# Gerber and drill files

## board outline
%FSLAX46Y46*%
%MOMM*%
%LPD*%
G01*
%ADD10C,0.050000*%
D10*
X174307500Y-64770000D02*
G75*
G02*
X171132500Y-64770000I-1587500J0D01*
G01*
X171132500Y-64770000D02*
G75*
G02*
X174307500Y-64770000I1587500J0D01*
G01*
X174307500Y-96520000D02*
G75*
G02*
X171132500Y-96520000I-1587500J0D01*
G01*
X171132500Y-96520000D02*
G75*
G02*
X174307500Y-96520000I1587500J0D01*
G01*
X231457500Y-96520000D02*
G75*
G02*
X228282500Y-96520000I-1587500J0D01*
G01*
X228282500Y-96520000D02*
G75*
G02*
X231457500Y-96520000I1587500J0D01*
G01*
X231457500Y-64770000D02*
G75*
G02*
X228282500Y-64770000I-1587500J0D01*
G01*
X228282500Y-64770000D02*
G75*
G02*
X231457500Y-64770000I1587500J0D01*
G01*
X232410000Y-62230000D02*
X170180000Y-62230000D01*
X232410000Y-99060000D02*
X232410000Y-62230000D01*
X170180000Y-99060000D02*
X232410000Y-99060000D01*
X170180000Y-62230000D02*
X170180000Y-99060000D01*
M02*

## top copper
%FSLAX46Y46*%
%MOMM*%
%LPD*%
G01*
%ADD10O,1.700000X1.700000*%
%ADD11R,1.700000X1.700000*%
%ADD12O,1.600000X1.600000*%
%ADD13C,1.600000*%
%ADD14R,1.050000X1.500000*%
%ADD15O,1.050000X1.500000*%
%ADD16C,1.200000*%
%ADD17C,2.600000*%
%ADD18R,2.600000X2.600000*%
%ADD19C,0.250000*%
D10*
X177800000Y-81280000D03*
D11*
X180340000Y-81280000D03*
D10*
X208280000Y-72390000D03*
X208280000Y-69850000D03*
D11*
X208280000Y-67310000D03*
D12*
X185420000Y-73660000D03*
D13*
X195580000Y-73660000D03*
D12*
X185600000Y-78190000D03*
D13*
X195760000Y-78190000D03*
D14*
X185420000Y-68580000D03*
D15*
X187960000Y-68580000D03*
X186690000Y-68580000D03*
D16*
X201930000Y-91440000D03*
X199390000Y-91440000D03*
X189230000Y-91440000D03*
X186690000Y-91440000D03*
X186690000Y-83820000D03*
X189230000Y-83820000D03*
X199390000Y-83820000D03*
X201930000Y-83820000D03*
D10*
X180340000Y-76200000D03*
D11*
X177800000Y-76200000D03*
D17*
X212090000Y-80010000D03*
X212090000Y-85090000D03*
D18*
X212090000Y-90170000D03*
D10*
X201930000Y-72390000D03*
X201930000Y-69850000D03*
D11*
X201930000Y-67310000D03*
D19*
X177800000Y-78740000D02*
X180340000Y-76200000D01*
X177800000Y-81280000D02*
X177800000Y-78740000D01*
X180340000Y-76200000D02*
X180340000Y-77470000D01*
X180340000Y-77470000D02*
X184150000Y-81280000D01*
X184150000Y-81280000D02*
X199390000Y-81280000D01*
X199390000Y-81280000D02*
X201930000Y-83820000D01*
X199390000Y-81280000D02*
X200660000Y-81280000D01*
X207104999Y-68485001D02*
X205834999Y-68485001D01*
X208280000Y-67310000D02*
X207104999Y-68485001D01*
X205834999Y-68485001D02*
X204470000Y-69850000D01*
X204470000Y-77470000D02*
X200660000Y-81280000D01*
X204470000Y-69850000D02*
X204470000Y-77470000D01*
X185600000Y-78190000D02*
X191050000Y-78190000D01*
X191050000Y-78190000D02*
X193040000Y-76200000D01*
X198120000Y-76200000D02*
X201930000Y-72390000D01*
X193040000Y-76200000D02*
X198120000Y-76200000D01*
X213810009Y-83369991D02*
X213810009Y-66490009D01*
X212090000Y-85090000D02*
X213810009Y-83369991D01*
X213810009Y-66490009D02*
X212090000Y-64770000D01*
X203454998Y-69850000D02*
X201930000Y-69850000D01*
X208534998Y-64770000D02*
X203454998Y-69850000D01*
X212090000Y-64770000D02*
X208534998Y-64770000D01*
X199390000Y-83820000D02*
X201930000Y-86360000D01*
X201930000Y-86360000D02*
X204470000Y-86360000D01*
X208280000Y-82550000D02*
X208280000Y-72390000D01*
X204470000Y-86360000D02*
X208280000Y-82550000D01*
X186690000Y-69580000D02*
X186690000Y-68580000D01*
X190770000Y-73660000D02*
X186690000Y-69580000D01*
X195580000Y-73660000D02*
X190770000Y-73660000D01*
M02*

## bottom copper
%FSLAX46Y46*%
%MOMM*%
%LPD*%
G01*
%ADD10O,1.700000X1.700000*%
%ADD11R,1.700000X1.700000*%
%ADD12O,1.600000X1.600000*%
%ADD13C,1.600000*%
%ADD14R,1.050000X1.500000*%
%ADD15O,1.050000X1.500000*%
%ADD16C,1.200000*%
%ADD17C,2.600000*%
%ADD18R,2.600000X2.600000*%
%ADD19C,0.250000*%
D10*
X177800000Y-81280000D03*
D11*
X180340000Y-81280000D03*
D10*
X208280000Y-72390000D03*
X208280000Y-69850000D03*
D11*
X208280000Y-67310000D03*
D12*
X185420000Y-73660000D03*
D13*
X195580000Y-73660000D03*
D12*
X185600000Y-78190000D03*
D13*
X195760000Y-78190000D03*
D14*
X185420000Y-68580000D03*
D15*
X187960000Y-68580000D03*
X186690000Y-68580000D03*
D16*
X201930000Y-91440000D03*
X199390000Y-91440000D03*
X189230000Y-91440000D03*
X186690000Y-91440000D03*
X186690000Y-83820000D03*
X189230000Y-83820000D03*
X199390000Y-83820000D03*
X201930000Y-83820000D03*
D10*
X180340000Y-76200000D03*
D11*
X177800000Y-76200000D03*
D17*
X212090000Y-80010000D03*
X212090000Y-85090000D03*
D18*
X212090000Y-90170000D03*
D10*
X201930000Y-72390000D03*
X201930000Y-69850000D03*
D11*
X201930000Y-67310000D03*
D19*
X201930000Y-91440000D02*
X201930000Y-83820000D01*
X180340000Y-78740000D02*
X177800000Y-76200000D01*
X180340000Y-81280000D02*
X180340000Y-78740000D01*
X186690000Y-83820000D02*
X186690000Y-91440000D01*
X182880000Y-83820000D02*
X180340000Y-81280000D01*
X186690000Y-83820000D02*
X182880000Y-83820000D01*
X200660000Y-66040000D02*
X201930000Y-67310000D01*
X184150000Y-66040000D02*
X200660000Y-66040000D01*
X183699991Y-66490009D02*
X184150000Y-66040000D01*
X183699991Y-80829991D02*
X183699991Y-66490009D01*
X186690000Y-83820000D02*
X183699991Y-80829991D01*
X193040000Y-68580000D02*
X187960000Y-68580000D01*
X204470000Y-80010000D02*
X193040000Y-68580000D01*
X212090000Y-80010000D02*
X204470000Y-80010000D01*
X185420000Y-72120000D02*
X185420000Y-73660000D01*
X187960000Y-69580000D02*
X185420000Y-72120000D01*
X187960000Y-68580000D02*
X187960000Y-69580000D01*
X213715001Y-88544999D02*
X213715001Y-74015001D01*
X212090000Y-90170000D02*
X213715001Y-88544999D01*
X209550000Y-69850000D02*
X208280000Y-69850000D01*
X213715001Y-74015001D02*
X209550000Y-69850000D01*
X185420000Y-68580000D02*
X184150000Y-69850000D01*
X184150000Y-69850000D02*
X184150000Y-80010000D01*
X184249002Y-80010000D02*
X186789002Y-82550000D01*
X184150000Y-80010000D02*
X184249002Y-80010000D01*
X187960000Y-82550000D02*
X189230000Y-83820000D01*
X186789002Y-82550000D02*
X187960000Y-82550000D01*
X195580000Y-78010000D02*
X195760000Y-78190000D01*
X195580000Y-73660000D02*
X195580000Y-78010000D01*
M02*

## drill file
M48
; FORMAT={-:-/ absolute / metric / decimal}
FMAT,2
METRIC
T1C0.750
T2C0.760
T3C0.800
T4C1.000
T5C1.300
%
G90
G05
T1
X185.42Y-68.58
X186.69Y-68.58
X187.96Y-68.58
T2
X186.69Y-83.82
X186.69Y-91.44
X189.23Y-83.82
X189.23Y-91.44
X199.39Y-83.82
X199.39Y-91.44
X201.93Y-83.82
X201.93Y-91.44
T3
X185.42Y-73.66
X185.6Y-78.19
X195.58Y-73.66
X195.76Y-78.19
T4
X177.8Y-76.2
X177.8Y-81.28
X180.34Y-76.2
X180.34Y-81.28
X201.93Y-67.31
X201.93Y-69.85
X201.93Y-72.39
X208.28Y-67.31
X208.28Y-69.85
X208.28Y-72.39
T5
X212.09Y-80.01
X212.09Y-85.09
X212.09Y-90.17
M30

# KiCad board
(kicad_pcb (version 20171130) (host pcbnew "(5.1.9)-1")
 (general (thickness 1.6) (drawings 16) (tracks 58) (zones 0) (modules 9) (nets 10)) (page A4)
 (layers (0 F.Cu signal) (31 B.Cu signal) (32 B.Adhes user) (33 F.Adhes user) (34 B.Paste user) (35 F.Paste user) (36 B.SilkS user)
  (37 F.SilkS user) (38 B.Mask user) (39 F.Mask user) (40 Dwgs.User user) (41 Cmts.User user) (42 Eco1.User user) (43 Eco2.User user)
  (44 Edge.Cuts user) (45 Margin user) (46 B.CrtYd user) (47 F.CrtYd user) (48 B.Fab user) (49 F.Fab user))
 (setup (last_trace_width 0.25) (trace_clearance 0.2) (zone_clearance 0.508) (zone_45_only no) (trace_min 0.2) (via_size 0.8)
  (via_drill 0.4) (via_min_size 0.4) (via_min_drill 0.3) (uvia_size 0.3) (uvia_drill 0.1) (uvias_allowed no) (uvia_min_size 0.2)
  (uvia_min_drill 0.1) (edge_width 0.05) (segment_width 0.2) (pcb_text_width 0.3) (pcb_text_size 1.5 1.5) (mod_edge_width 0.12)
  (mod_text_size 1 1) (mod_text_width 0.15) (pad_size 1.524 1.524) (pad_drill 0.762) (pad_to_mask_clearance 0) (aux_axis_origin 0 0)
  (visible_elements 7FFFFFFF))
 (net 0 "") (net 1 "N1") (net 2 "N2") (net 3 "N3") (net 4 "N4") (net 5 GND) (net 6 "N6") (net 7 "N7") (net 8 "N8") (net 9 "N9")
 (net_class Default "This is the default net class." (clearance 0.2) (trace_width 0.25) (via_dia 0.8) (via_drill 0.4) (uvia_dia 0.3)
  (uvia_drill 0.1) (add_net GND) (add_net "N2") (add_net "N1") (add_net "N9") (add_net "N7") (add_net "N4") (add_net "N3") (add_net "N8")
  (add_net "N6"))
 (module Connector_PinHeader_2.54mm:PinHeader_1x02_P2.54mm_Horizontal (layer F.Cu) (at 180.34 81.28 270)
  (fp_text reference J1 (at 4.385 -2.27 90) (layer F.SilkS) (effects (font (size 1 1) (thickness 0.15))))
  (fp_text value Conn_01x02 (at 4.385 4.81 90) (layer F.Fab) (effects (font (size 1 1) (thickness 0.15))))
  (pad 2 thru_hole oval (at 0 2.54 270) (size 1.7 1.7) (drill 1) (layers *.Cu *.Mask) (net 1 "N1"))
  (pad 1 thru_hole rect (at 0 0 270) (size 1.7 1.7) (drill 1) (layers *.Cu *.Mask) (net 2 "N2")))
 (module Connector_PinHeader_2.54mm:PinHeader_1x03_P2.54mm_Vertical (layer F.Cu) (at 208.28 67.31)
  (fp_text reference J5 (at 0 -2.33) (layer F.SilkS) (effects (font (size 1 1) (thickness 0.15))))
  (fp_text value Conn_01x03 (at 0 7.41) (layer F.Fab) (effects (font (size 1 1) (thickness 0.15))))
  (pad 3 thru_hole oval (at 0 5.08) (size 1.7 1.7) (drill 1) (layers *.Cu *.Mask) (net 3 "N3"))
  (pad 2 thru_hole oval (at 0 2.54) (size 1.7 1.7) (drill 1) (layers *.Cu *.Mask) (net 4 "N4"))
  (pad 1 thru_hole rect (at 0 0) (size 1.7 1.7) (drill 1) (layers *.Cu *.Mask) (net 1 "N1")))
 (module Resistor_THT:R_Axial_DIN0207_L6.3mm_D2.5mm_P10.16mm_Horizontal (layer F.Cu) (at 195.58 73.66 180)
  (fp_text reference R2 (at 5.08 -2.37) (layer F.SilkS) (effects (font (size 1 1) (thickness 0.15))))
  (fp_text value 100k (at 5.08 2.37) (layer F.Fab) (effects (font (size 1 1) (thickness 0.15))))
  (pad 2 thru_hole oval (at 10.16 0 180) (size 1.6 1.6) (drill 0.8) (layers *.Cu *.Mask) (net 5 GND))
  (pad 1 thru_hole circle (at 0 0 180) (size 1.6 1.6) (drill 0.8) (layers *.Cu *.Mask) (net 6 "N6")))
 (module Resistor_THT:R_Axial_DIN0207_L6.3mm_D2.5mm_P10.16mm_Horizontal (layer F.Cu) (at 195.76 78.19 180)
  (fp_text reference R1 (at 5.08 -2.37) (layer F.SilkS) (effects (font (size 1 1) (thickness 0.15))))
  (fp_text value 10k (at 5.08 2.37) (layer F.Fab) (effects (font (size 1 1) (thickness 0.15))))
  (pad 2 thru_hole oval (at 10.16 0 180) (size 1.6 1.6) (drill 0.8) (layers *.Cu *.Mask) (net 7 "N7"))
  (pad 1 thru_hole circle (at 0 0 180) (size 1.6 1.6) (drill 0.8) (layers *.Cu *.Mask) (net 6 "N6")))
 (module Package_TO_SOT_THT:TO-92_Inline (layer F.Cu) (at 185.42 68.58)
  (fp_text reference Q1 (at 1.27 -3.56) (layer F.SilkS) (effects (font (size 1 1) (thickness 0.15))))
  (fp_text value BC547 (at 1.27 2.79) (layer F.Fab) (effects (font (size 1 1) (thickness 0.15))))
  (pad 1 thru_hole rect (at 0 0) (size 1.05 1.5) (drill 0.75) (layers *.Cu *.Mask) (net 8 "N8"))
  (pad 3 thru_hole oval (at 2.54 0) (size 1.05 1.5) (drill 0.75) (layers *.Cu *.Mask) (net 5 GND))
  (pad 2 thru_hole oval (at 1.27 0) (size 1.05 1.5) (drill 0.75) (layers *.Cu *.Mask) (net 6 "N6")))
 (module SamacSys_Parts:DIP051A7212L (layer F.Cu) (at 201.93 83.82 180)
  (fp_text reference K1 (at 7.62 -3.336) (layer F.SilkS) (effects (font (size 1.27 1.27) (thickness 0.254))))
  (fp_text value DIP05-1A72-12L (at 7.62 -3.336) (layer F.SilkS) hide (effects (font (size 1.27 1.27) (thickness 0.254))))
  (pad 14 thru_hole circle (at 0 -7.62 180) (size 1.2 1.2) (drill 0.76) (layers *.Cu *.Mask) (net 1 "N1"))
  (pad 13 thru_hole circle (at 2.54 -7.62 180) (size 1.2 1.2) (drill 0.76) (layers *.Cu *.Mask))
  (pad 9 thru_hole circle (at 12.7 -7.62 180) (size 1.2 1.2) (drill 0.76) (layers *.Cu *.Mask))
  (pad 8 thru_hole circle (at 15.24 -7.62 180) (size 1.2 1.2) (drill 0.76) (layers *.Cu *.Mask) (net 2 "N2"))
  (pad 7 thru_hole circle (at 15.24 0 180) (size 1.2 1.2) (drill 0.76) (layers *.Cu *.Mask) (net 2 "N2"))
  (pad 6 thru_hole circle (at 12.7 0 180) (size 1.2 1.2) (drill 0.76) (layers *.Cu *.Mask) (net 8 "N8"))
  (pad 2 thru_hole circle (at 2.54 0 180) (size 1.2 1.2) (drill 0.76) (layers *.Cu *.Mask) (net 3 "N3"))
  (pad 1 thru_hole circle (at 0 0 180) (size 1.2 1.2) (drill 0.76) (layers *.Cu *.Mask) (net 1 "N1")))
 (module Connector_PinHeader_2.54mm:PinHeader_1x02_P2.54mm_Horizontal (layer F.Cu) (at 177.8 76.2 90)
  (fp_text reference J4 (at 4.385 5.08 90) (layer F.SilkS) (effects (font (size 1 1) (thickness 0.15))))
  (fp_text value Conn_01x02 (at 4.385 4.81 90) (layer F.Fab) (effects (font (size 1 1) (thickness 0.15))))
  (pad 2 thru_hole oval (at 0 2.54 90) (size 1.7 1.7) (drill 1) (layers *.Cu *.Mask) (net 1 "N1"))
  (pad 1 thru_hole rect (at 0 0 90) (size 1.7 1.7) (drill 1) (layers *.Cu *.Mask) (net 2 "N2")))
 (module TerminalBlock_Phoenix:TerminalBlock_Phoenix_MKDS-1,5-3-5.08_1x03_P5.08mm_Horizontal (layer F.Cu) (at 212.09 90.17 90)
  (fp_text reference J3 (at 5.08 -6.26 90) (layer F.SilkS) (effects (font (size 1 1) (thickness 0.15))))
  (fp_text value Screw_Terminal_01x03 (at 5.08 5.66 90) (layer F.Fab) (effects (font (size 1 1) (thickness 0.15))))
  (pad 3 thru_hole circle (at 10.16 0 90) (size 2.6 2.6) (drill 1.3) (layers *.Cu *.Mask) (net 5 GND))
  (pad 2 thru_hole circle (at 5.08 0 90) (size 2.6 2.6) (drill 1.3) (layers *.Cu *.Mask) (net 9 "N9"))
  (pad 1 thru_hole rect (at 0 0 90) (size 2.6 2.6) (drill 1.3) (layers *.Cu *.Mask) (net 4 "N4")))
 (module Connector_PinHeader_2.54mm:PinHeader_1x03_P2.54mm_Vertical (layer F.Cu) (at 201.93 67.31)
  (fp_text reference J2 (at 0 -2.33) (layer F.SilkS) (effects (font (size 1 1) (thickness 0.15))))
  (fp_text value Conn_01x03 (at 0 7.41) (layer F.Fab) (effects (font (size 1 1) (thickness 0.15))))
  (pad 3 thru_hole oval (at 0 5.08) (size 1.7 1.7) (drill 1) (layers *.Cu *.Mask) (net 7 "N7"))
  (pad 2 thru_hole oval (at 0 2.54) (size 1.7 1.7) (drill 1) (layers *.Cu *.Mask) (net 9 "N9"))
  (pad 1 thru_hole rect (at 0 0) (size 1.7 1.7) (drill 1) (layers *.Cu *.Mask) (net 2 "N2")))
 (gr_circle (center 172.72 64.77) (end 174.3075 64.77) (layer Edge.Cuts) (width 0.05))
 (gr_circle (center 172.72 96.52) (end 174.3075 96.52) (layer Edge.Cuts) (width 0.05))
 (gr_circle (center 229.87 96.52) (end 231.4575 96.52) (layer Edge.Cuts) (width 0.05))
 (gr_circle (center 229.87 64.77) (end 231.4575 64.77) (layer Edge.Cuts) (width 0.05))
 (gr_line (start 232.41 62.23) (end 170.18 62.23) (layer Edge.Cuts) (width 0.05))
 (gr_line (start 232.41 99.06) (end 232.41 62.23) (layer Edge.Cuts) (width 0.05))
 (gr_line (start 170.18 99.06) (end 232.41 99.06) (layer Edge.Cuts) (width 0.05))
 (gr_line (start 170.18 62.23) (end 170.18 99.06) (layer Edge.Cuts) (width 0.05))
 (segment (start 177.8 78.74) (end 180.34 76.2) (width 0.25) (layer F.Cu) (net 1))
 (segment (start 177.8 81.28) (end 177.8 78.74) (width 0.25) (layer F.Cu) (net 1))
 (segment (start 201.93 91.44) (end 201.93 83.82) (width 0.25) (layer B.Cu) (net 1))
 (segment (start 180.34 76.2) (end 180.34 77.47) (width 0.25) (layer F.Cu) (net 1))
 (segment (start 180.34 77.47) (end 184.15 81.28) (width 0.25) (layer F.Cu) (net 1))
 (segment (start 184.15 81.28) (end 199.39 81.28) (width 0.25) (layer F.Cu) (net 1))
 (segment (start 199.39 81.28) (end 201.93 83.82) (width 0.25) (layer F.Cu) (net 1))
 (segment (start 199.39 81.28) (end 200.66 81.28) (width 0.25) (layer F.Cu) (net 1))
 (segment (start 207.104999 68.485001) (end 205.834999 68.485001) (width 0.25) (layer F.Cu) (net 1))
 (segment (start 208.28 67.31) (end 207.104999 68.485001) (width 0.25) (layer F.Cu) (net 1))
 (segment (start 205.834999 68.485001) (end 204.47 69.85) (width 0.25) (layer F.Cu) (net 1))
 (segment (start 204.47 77.47) (end 200.66 81.28) (width 0.25) (layer F.Cu) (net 1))
 (segment (start 204.47 69.85) (end 204.47 77.47) (width 0.25) (layer F.Cu) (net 1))
 (segment (start 180.34 78.74) (end 177.8 76.2) (width 0.25) (layer B.Cu) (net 2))
 (segment (start 180.34 81.28) (end 180.34 78.74) (width 0.25) (layer B.Cu) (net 2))
 (segment (start 186.69 83.82) (end 186.69 91.44) (width 0.25) (layer B.Cu) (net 2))
 (segment (start 182.88 83.82) (end 180.34 81.28) (width 0.25) (layer B.Cu) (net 2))
 (segment (start 186.69 83.82) (end 182.88 83.82) (width 0.25) (layer B.Cu) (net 2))
 (segment (start 200.66 66.04) (end 201.93 67.31) (width 0.25) (layer B.Cu) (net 2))
 (segment (start 184.15 66.04) (end 200.66 66.04) (width 0.25) (layer B.Cu) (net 2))
 (segment (start 183.699991 66.490009) (end 184.15 66.04) (width 0.25) (layer B.Cu) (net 2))
 (segment (start 183.699991 80.829991) (end 183.699991 66.490009) (width 0.25) (layer B.Cu) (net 2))
 (segment (start 186.69 83.82) (end 183.699991 80.829991) (width 0.25) (layer B.Cu) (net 2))
 (segment (start 185.6 78.19) (end 191.05 78.19) (width 0.25) (layer F.Cu) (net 7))
 (segment (start 191.05 78.19) (end 193.04 76.2) (width 0.25) (layer F.Cu) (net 7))
 (segment (start 198.12 76.2) (end 201.93 72.39) (width 0.25) (layer F.Cu) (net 7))
 (segment (start 193.04 76.2) (end 198.12 76.2) (width 0.25) (layer F.Cu) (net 7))
 (segment (start 213.810009 83.369991) (end 213.810009 66.490009) (width 0.25) (layer F.Cu) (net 9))
 (segment (start 212.09 85.09) (end 213.810009 83.369991) (width 0.25) (layer F.Cu) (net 9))
 (segment (start 213.810009 66.490009) (end 212.09 64.77) (width 0.25) (layer F.Cu) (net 9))
 (segment (start 203.454998 69.85) (end 201.93 69.85) (width 0.25) (layer F.Cu) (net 9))
 (segment (start 208.534998 64.77) (end 203.454998 69.85) (width 0.25) (layer F.Cu) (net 9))
 (segment (start 212.09 64.77) (end 208.534998 64.77) (width 0.25) (layer F.Cu) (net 9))
 (segment (start 193.04 68.58) (end 187.96 68.58) (width 0.25) (layer B.Cu) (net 5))
 (segment (start 204.47 80.01) (end 193.04 68.58) (width 0.25) (layer B.Cu) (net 5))
 (segment (start 212.09 80.01) (end 204.47 80.01) (width 0.25) (layer B.Cu) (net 5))
 (segment (start 185.42 72.12) (end 185.42 73.66) (width 0.25) (layer B.Cu) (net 5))
 (segment (start 187.96 69.58) (end 185.42 72.12) (width 0.25) (layer B.Cu) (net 5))
 (segment (start 187.96 68.58) (end 187.96 69.58) (width 0.25) (layer B.Cu) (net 5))
 (segment (start 213.715001 88.544999) (end 213.715001 74.015001) (width 0.25) (layer B.Cu) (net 4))
 (segment (start 212.09 90.17) (end 213.715001 88.544999) (width 0.25) (layer B.Cu) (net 4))
 (segment (start 209.55 69.85) (end 208.28 69.85) (width 0.25) (layer B.Cu) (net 4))
 (segment (start 213.715001 74.015001) (end 209.55 69.85) (width 0.25) (layer B.Cu) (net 4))
 (segment (start 185.42 68.58) (end 184.15 69.85) (width 0.25) (layer B.Cu) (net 8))
 (segment (start 184.15 69.85) (end 184.15 80.01) (width 0.25) (layer B.Cu) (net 8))
 (segment (start 184.249002 80.01) (end 186.789002 82.55) (width 0.25) (layer B.Cu) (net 8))
 (segment (start 184.15 80.01) (end 184.249002 80.01) (width 0.25) (layer B.Cu) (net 8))
 (segment (start 187.96 82.55) (end 189.23 83.82) (width 0.25) (layer B.Cu) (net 8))
 (segment (start 186.789002 82.55) (end 187.96 82.55) (width 0.25) (layer B.Cu) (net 8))
 (segment (start 199.39 83.82) (end 201.93 86.36) (width 0.25) (layer F.Cu) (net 3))
 (segment (start 201.93 86.36) (end 204.47 86.36) (width 0.25) (layer F.Cu) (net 3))
 (segment (start 208.28 82.55) (end 208.28 72.39) (width 0.25) (layer F.Cu) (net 3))
 (segment (start 204.47 86.36) (end 208.28 82.55) (width 0.25) (layer F.Cu) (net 3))
 (segment (start 186.69 69.58) (end 186.69 68.58) (width 0.25) (layer F.Cu) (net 6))
 (segment (start 190.77 73.66) (end 186.69 69.58) (width 0.25) (layer F.Cu) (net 6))
 (segment (start 195.58 73.66) (end 190.77 73.66) (width 0.25) (layer F.Cu) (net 6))
 (segment (start 195.58 78.01) (end 195.76 78.19) (width 0.25) (layer B.Cu) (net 6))
 (segment (start 195.58 73.66) (end 195.58 78.01) (width 0.25) (layer B.Cu) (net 6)))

